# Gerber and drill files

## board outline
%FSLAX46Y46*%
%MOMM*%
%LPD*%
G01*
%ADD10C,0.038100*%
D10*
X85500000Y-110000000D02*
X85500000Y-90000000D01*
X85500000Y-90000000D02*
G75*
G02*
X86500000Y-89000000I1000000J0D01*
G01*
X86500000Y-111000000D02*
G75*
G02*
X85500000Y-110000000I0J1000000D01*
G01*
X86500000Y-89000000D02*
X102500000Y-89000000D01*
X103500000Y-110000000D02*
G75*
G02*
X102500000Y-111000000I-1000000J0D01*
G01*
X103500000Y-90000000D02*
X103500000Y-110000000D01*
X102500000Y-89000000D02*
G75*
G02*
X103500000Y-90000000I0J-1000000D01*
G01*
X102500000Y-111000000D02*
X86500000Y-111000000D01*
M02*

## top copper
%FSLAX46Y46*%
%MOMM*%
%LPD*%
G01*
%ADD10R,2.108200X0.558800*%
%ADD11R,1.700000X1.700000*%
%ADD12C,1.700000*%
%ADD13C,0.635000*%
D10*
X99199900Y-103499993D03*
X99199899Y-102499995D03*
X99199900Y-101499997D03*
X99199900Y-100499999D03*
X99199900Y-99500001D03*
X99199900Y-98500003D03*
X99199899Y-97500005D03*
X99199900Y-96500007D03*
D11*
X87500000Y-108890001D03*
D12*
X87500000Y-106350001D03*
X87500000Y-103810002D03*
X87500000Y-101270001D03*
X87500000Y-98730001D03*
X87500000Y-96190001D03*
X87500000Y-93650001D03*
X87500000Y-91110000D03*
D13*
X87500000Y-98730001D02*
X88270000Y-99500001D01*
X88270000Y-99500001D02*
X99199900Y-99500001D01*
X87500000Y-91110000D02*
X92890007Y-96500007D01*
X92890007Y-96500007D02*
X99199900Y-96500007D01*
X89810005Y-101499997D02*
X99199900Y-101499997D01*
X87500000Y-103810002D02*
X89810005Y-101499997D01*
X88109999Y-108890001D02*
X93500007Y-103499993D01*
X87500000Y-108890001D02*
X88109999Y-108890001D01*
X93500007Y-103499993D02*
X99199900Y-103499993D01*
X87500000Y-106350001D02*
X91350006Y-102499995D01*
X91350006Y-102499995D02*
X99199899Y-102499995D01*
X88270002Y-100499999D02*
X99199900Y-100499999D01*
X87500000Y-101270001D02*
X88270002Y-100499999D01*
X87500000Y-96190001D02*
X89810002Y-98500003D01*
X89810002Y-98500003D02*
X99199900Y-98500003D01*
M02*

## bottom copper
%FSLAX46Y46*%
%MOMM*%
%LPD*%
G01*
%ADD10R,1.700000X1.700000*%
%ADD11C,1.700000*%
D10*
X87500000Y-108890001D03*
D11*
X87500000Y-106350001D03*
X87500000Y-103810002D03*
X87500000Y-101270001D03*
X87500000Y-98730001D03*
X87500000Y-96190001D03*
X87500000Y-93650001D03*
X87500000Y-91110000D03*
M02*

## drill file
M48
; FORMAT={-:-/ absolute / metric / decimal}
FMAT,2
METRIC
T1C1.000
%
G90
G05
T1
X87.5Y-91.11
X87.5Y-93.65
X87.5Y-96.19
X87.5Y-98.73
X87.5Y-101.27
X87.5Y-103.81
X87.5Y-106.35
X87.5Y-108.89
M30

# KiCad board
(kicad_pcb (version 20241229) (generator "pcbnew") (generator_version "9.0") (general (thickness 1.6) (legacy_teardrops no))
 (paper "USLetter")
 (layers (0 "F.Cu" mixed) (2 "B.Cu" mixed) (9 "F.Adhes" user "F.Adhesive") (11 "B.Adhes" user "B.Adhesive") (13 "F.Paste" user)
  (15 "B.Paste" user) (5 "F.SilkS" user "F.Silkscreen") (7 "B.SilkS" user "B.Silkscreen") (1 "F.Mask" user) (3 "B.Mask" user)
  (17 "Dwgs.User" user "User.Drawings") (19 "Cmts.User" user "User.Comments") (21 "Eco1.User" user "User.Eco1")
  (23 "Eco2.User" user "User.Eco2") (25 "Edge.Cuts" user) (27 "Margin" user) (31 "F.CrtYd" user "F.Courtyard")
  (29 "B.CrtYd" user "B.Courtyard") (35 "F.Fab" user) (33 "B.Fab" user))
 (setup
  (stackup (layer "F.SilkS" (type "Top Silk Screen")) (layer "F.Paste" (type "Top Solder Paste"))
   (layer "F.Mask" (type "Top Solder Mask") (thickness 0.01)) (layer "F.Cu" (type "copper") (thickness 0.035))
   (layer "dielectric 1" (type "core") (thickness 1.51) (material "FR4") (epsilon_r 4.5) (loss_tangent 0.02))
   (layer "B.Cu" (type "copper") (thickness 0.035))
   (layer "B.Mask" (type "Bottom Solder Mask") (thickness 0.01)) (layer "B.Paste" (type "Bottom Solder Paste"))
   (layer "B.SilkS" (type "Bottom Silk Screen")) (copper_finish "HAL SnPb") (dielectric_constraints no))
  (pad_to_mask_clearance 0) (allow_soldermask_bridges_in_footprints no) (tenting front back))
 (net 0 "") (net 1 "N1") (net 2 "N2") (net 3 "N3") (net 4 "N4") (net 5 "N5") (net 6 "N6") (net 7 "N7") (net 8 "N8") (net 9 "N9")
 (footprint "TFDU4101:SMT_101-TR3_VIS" (layer "F.Cu") (at 100 100)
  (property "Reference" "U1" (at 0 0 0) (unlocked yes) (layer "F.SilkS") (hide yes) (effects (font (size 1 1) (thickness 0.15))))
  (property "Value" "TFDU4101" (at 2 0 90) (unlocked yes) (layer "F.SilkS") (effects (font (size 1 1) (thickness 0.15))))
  (pad "1" smd rect (at -0.8001 3.499993) (size 2.1082 0.5588) (layers "F.Cu" "F.Mask" "F.Paste") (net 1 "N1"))
  (pad "2" smd rect (at -0.800101 2.499995) (size 2.1082 0.5588) (layers "F.Cu" "F.Mask" "F.Paste") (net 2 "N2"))
  (pad "3" smd rect (at -0.8001 1.499997) (size 2.1082 0.5588) (layers "F.Cu" "F.Mask" "F.Paste") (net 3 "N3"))
  (pad "4" smd rect (at -0.8001 0.499999) (size 2.1082 0.5588) (layers "F.Cu" "F.Mask" "F.Paste") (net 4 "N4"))
  (pad "5" smd rect (at -0.8001 -0.499999) (size 2.1082 0.5588) (layers "F.Cu" "F.Mask" "F.Paste") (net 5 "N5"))
  (pad "6" smd rect (at -0.8001 -1.499997) (size 2.1082 0.5588) (layers "F.Cu" "F.Mask" "F.Paste") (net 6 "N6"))
  (pad "7" smd rect (at -0.800101 -2.499995) (size 2.1082 0.5588) (layers "F.Cu" "F.Mask" "F.Paste") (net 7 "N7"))
  (pad "8" smd rect (at -0.8001 -3.499993) (size 2.1082 0.5588) (layers "F.Cu" "F.Mask" "F.Paste") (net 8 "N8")))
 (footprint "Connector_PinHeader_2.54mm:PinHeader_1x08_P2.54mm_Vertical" (layer "B.Cu") (at 87.5 108.890001)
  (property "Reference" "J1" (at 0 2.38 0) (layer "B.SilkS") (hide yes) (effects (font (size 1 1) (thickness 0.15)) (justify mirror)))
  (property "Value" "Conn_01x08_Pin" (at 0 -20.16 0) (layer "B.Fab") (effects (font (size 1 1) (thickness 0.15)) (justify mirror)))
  (pad "1" thru_hole rect (at 0 0) (size 1.7 1.7) (drill 1) (layers "*.Cu" "*.Mask") (remove_unused_layers no) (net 1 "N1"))
  (pad "2" thru_hole circle (at 0 -2.54) (size 1.7 1.7) (drill 1) (layers "*.Cu" "*.Mask") (remove_unused_layers no) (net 2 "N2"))
  (pad "3" thru_hole circle (at 0 -5.079999) (size 1.7 1.7) (drill 1) (layers "*.Cu" "*.Mask") (remove_unused_layers no) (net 3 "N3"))
  (pad "4" thru_hole circle (at 0 -7.62) (size 1.7 1.7) (drill 1) (layers "*.Cu" "*.Mask") (remove_unused_layers no) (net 4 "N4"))
  (pad "5" thru_hole circle (at 0 -10.16) (size 1.7 1.7) (drill 1) (layers "*.Cu" "*.Mask") (remove_unused_layers no) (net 5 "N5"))
  (pad "6" thru_hole circle (at 0 -12.7) (size 1.7 1.7) (drill 1) (layers "*.Cu" "*.Mask") (remove_unused_layers no) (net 6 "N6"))
  (pad "7" thru_hole circle (at 0 -15.24) (size 1.7 1.7) (drill 1) (layers "*.Cu" "*.Mask") (remove_unused_layers no) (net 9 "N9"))
  (pad "8" thru_hole circle (at 0 -17.780001) (size 1.7 1.7) (drill 1) (layers "*.Cu" "*.Mask") (remove_unused_layers no) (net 8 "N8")))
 (gr_line (start 85.5 110) (end 85.5 90) (stroke (width 0.0381) (type default)) (layer "Edge.Cuts"))
 (gr_arc (start 85.5 90) (mid 85.792893 89.292893) (end 86.5 89) (stroke (width 0.0381) (type default)) (layer "Edge.Cuts"))
 (gr_arc (start 86.5 111) (mid 85.792893 110.707107) (end 85.5 110) (stroke (width 0.0381) (type default)) (layer "Edge.Cuts"))
 (gr_line (start 86.5 89) (end 102.5 89) (stroke (width 0.0381) (type default)) (layer "Edge.Cuts"))
 (gr_arc (start 103.5 110) (mid 103.207107 110.707107) (end 102.5 111) (stroke (width 0.0381) (type default)) (layer "Edge.Cuts"))
 (gr_line (start 103.5 90) (end 103.5 110) (stroke (width 0.0381) (type default)) (layer "Edge.Cuts"))
 (gr_arc (start 102.5 89) (mid 103.207107 89.292893) (end 103.5 90) (stroke (width 0.0381) (type default)) (layer "Edge.Cuts"))
 (gr_line (start 102.5 111) (end 86.5 111) (stroke (width 0.0381) (type default)) (layer "Edge.Cuts"))
 (segment (start 87.5 98.730001) (end 88.27 99.500001) (width 0.635) (layer "F.Cu") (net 5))
 (segment (start 88.27 99.500001) (end 99.1999 99.500001) (width 0.635) (layer "F.Cu") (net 5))
 (segment (start 87.5 91.11) (end 92.890007 96.500007) (width 0.635) (layer "F.Cu") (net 8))
 (segment (start 92.890007 96.500007) (end 99.1999 96.500007) (width 0.635) (layer "F.Cu") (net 8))
 (segment (start 89.810005 101.499997) (end 99.1999 101.499997) (width 0.635) (layer "F.Cu") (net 3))
 (segment (start 87.5 103.810002) (end 89.810005 101.499997) (width 0.635) (layer "F.Cu") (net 3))
 (segment (start 88.109999 108.890001) (end 93.500007 103.499993) (width 0.635) (layer "F.Cu") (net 1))
 (segment (start 87.5 108.890001) (end 88.109999 108.890001) (width 0.635) (layer "F.Cu") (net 1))
 (segment (start 93.500007 103.499993) (end 99.1999 103.499993) (width 0.635) (layer "F.Cu") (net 1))
 (segment (start 87.5 106.350001) (end 91.350006 102.499995) (width 0.635) (layer "F.Cu") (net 2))
 (segment (start 91.350006 102.499995) (end 99.199899 102.499995) (width 0.635) (layer "F.Cu") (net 2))
 (segment (start 88.270002 100.499999) (end 99.1999 100.499999) (width 0.635) (layer "F.Cu") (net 4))
 (segment (start 87.5 101.270001) (end 88.270002 100.499999) (width 0.635) (layer "F.Cu") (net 4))
 (segment (start 87.5 96.190001) (end 89.810002 98.500003) (width 0.635) (layer "F.Cu") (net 6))
 (segment (start 89.810002 98.500003) (end 99.1999 98.500003) (width 0.635) (layer "F.Cu") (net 6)))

